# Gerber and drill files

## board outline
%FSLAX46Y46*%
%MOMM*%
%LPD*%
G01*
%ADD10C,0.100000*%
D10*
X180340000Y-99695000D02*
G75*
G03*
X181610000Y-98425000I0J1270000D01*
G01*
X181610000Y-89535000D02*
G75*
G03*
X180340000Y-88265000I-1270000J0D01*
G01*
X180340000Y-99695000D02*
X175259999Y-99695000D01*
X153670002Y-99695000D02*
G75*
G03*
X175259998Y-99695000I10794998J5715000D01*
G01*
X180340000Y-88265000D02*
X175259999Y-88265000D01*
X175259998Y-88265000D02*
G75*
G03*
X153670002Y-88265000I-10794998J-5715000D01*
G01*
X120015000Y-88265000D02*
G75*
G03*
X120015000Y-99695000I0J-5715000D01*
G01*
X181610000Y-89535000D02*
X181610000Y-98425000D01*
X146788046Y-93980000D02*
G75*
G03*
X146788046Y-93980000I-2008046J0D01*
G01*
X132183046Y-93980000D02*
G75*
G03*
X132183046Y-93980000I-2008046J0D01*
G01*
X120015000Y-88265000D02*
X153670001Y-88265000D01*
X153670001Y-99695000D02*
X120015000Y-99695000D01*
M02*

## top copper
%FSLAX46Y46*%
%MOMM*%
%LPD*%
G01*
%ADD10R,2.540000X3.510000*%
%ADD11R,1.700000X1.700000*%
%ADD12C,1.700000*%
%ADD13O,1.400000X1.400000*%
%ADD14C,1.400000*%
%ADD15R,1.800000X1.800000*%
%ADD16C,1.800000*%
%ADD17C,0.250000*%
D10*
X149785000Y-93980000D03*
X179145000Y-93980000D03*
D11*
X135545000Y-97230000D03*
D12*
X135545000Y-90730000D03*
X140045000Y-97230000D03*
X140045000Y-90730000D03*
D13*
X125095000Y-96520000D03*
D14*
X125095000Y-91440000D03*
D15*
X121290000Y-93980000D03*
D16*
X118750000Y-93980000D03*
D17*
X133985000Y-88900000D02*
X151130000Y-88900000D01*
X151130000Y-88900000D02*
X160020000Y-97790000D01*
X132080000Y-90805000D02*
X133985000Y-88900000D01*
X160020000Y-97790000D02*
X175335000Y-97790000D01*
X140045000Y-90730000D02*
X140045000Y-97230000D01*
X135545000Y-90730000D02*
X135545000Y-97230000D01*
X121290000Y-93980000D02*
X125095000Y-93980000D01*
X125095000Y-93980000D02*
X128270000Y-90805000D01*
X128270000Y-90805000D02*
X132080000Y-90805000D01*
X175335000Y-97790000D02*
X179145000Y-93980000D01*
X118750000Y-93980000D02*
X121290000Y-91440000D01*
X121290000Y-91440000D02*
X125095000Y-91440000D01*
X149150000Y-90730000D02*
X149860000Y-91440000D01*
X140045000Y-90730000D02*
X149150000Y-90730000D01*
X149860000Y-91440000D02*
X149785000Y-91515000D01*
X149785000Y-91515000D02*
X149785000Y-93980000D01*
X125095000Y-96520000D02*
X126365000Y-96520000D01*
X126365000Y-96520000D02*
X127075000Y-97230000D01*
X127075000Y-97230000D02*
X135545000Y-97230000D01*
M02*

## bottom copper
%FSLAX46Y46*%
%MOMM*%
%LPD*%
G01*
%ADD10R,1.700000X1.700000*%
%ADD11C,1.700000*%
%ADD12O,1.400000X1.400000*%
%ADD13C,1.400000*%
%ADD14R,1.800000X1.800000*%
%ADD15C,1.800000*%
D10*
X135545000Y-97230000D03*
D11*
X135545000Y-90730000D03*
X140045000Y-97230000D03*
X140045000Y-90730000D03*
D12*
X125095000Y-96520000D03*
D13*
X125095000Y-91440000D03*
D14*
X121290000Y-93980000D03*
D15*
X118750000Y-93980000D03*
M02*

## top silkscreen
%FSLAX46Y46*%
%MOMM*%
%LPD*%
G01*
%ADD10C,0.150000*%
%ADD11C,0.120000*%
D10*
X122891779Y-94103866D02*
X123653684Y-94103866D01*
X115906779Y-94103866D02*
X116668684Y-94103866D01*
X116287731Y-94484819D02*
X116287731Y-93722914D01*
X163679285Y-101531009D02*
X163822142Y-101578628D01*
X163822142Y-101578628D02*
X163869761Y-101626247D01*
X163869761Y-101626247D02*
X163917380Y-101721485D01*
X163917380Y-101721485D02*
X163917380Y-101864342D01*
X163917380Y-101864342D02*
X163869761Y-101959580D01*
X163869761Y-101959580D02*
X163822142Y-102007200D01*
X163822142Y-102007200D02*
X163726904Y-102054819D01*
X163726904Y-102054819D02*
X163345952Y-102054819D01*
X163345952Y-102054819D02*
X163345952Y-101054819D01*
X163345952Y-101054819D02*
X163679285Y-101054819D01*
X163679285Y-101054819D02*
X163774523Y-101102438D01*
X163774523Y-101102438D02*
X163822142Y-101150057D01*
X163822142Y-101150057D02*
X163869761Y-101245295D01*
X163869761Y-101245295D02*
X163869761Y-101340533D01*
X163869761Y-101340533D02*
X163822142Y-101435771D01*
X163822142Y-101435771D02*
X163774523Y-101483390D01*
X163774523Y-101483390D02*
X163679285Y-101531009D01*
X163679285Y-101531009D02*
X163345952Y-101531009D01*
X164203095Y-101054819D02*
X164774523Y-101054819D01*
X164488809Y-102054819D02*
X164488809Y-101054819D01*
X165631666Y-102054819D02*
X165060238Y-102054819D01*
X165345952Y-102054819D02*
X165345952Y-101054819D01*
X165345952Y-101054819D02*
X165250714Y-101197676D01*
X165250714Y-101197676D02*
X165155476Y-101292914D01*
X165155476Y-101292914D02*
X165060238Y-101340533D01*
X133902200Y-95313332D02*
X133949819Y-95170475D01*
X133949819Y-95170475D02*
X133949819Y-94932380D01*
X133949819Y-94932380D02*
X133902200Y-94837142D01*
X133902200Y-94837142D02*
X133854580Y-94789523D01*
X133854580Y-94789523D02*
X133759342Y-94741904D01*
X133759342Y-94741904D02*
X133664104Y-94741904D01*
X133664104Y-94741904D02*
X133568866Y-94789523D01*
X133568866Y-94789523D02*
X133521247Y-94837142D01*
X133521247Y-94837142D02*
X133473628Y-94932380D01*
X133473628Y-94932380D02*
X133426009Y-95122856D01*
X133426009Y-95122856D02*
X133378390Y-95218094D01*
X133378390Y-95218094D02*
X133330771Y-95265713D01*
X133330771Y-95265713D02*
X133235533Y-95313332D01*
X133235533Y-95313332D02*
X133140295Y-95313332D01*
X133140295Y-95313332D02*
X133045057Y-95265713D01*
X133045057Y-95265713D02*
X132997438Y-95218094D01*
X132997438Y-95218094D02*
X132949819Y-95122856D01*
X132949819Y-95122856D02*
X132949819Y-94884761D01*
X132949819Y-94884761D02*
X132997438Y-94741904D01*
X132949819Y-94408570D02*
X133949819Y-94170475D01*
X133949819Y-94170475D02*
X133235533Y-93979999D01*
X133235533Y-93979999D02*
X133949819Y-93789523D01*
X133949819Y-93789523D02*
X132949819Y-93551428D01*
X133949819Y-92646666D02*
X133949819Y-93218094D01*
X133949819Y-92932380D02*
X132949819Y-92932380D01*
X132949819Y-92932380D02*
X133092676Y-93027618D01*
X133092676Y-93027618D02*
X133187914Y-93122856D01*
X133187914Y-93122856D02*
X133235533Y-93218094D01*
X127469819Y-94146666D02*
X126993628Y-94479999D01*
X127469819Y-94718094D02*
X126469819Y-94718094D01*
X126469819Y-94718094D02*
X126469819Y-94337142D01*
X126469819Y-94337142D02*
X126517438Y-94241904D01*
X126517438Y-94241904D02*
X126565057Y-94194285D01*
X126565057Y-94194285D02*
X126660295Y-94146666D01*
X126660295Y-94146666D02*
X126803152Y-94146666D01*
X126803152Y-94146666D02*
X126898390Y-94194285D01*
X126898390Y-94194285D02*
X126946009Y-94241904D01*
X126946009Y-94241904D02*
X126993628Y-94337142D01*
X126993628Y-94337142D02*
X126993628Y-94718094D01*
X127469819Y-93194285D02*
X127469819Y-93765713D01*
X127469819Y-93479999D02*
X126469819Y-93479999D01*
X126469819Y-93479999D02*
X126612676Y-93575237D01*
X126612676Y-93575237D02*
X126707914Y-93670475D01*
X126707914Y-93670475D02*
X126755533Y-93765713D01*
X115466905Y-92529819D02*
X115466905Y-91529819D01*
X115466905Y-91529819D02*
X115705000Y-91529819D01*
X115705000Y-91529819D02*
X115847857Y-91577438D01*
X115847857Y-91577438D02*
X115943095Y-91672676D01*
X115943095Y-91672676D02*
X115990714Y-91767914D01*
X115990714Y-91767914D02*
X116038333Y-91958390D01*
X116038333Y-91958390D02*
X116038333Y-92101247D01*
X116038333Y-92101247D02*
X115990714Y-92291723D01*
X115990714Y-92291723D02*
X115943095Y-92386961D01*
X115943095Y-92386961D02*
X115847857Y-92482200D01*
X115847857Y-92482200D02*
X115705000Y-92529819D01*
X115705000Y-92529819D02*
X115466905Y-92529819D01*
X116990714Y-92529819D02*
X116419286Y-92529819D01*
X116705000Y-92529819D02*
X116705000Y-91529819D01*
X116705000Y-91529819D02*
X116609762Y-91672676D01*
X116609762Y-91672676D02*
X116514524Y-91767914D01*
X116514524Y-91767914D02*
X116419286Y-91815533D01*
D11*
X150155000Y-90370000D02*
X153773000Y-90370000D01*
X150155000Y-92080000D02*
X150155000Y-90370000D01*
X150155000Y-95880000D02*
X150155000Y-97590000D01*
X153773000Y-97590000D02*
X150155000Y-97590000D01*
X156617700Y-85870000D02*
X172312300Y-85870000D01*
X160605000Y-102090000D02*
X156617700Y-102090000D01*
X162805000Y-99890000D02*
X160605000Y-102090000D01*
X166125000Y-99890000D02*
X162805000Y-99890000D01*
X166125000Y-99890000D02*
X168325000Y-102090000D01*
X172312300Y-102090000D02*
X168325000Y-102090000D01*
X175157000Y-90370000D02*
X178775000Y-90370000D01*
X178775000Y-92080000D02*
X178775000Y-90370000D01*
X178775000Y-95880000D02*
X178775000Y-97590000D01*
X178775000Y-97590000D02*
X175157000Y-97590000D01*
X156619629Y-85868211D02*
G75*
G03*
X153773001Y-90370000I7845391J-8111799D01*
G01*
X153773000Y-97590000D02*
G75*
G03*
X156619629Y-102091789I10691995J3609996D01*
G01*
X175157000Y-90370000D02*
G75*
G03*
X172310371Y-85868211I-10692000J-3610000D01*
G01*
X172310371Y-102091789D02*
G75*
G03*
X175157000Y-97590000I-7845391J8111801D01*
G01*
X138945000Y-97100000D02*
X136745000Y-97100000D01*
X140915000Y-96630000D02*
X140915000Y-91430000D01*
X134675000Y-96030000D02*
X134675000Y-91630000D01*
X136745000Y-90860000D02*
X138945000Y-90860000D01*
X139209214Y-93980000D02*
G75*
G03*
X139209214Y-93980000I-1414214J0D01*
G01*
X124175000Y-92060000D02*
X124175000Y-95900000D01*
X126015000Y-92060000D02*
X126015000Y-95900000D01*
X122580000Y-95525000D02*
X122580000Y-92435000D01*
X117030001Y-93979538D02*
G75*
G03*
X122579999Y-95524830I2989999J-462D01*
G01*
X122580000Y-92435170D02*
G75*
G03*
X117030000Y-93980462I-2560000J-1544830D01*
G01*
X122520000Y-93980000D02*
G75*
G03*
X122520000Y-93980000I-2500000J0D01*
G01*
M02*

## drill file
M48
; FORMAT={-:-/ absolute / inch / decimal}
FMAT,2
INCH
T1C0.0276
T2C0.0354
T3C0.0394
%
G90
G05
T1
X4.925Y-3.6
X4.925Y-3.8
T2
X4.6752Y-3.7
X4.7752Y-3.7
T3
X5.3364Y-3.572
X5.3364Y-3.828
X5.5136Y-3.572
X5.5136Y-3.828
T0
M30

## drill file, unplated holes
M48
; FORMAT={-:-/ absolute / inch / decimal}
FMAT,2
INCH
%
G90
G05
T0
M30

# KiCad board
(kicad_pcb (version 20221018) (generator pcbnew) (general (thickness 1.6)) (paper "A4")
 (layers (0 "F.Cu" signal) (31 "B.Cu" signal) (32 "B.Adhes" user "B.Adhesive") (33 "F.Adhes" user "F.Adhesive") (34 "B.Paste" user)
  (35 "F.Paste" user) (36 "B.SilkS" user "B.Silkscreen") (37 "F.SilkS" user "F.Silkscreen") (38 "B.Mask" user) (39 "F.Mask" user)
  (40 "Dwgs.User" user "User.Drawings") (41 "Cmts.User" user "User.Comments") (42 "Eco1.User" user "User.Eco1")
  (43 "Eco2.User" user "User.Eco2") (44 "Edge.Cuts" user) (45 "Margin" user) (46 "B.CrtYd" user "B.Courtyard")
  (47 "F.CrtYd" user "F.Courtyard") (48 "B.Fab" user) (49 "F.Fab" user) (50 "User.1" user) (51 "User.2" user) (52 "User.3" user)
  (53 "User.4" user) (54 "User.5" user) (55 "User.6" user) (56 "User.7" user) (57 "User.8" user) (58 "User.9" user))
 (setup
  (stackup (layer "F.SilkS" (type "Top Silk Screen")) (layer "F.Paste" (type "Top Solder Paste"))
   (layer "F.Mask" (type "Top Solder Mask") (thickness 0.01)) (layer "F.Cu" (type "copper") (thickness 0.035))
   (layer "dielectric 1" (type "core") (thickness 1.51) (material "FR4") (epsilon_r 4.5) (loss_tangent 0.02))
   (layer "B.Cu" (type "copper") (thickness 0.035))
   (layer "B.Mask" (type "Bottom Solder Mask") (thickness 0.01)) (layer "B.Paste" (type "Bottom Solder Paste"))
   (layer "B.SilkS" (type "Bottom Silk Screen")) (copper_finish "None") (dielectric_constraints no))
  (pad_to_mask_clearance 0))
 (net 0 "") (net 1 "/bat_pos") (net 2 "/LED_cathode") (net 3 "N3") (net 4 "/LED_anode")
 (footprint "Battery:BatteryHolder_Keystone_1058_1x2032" (layer "F.Cu") (at 164.465 93.98)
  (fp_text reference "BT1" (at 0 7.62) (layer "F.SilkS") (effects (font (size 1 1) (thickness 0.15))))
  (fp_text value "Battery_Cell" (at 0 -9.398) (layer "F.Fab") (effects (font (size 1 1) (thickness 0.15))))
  (fp_line (start -14.31 -3.61) (end -10.692 -3.61) (stroke (width 0.12) (type solid)) (layer "F.SilkS"))
  (fp_line (start -14.31 -1.9) (end -14.31 -3.61) (stroke (width 0.12) (type solid)) (layer "F.SilkS"))
  (fp_line (start -14.31 1.9) (end -14.31 3.61) (stroke (width 0.12) (type solid)) (layer "F.SilkS"))
  (fp_line (start -10.692 3.61) (end -14.31 3.61) (stroke (width 0.12) (type solid)) (layer "F.SilkS"))
  (fp_line (start -7.8473 -8.11) (end 7.8473 -8.11) (stroke (width 0.12) (type solid)) (layer "F.SilkS"))
  (fp_line (start -3.86 8.11) (end -7.8473 8.11) (stroke (width 0.12) (type solid)) (layer "F.SilkS"))
  (fp_line (start -1.66 5.91) (end -3.86 8.11) (stroke (width 0.12) (type solid)) (layer "F.SilkS"))
  (fp_line (start 1.66 5.91) (end -1.66 5.91) (stroke (width 0.12) (type solid)) (layer "F.SilkS"))
  (fp_line (start 1.66 5.91) (end 3.86 8.11) (stroke (width 0.12) (type solid)) (layer "F.SilkS"))
  (fp_line (start 7.8473 8.11) (end 3.86 8.11) (stroke (width 0.12) (type solid)) (layer "F.SilkS"))
  (fp_line (start 10.692 -3.61) (end 14.31 -3.61) (stroke (width 0.12) (type solid)) (layer "F.SilkS"))
  (fp_line (start 14.31 -1.9) (end 14.31 -3.61) (stroke (width 0.12) (type solid)) (layer "F.SilkS"))
  (fp_line (start 14.31 1.9) (end 14.31 3.61) (stroke (width 0.12) (type solid)) (layer "F.SilkS"))
  (fp_line (start 14.31 3.61) (end 10.692 3.61) (stroke (width 0.12) (type solid)) (layer "F.SilkS"))
  (fp_arc (start -10.692 -3.61) (mid -9.538084 -6.031244) (end -7.845371 -8.111789) (stroke (width 0.12) (type solid)) (layer "F.SilkS"))
  (fp_arc (start -7.845371 8.111789) (mid -9.538085 6.031244) (end -10.692 3.61) (stroke (width 0.12) (type solid)) (layer "F.SilkS"))
  (fp_arc (start 7.845371 -8.111789) (mid 9.538085 -6.031244) (end 10.692 -3.61) (stroke (width 0.12) (type solid)) (layer "F.SilkS"))
  (fp_arc (start 10.692 3.61) (mid 9.538084 6.031244) (end 7.845371 8.111789) (stroke (width 0.12) (type solid)) (layer "F.SilkS"))
  (pad "1" smd rect (at -14.68 0) (size 2.54 3.51) (layers "F.Cu" "F.Paste" "F.Mask") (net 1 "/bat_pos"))
  (pad "2" smd rect (at 14.68 0) (size 2.54 3.51) (layers "F.Cu" "F.Paste" "F.Mask") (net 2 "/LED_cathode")))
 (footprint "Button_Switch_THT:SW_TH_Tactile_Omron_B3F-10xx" (layer "F.Cu") (at 135.545 97.23 90)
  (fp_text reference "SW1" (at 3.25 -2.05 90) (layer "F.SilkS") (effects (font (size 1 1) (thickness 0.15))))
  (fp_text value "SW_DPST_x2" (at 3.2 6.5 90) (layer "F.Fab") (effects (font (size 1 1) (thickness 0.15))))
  (fp_line (start 0.13 3.4) (end 0.13 1.2) (stroke (width 0.12) (type solid)) (layer "F.SilkS"))
  (fp_line (start 0.6 5.37) (end 5.8 5.37) (stroke (width 0.12) (type solid)) (layer "F.SilkS"))
  (fp_line (start 1.2 -0.87) (end 5.6 -0.87) (stroke (width 0.12) (type solid)) (layer "F.SilkS"))
  (fp_line (start 6.37 1.2) (end 6.37 3.4) (stroke (width 0.12) (type solid)) (layer "F.SilkS"))
  (fp_circle (center 3.25 2.25) (end 4.25 3.25) (stroke (width 0.12) (type solid)) (fill none) (layer "F.SilkS"))
  (pad "1" thru_hole rect (at 0 0 90) (size 1.7 1.7) (drill 1) (layers "*.Cu" "*.Mask") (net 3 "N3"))
  (pad "1" thru_hole circle (at 6.5 0 90) (size 1.7 1.7) (drill 1) (layers "*.Cu" "*.Mask") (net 3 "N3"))
  (pad "2" thru_hole circle (at 0 4.5 90) (size 1.7 1.7) (drill 1) (layers "*.Cu" "*.Mask") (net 1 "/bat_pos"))
  (pad "2" thru_hole circle (at 6.5 4.5 90) (size 1.7 1.7) (drill 1) (layers "*.Cu" "*.Mask") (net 1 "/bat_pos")))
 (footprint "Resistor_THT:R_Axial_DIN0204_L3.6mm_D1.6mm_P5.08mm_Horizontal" (layer "F.Cu") (at 125.095 91.44 -90)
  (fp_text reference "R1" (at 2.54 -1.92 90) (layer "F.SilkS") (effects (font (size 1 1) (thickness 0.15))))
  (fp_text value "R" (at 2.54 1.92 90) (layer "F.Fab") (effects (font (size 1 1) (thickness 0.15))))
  (fp_line (start 0.62 -0.92) (end 4.46 -0.92) (stroke (width 0.12) (type solid)) (layer "F.SilkS"))
  (fp_line (start 0.62 0.92) (end 4.46 0.92) (stroke (width 0.12) (type solid)) (layer "F.SilkS"))
  (pad "1" thru_hole circle (at 0 0 270) (size 1.4 1.4) (drill 0.7) (layers "*.Cu" "*.Mask") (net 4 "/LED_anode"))
  (pad "2" thru_hole oval (at 5.08 0 270) (size 1.4 1.4) (drill 0.7) (layers "*.Cu" "*.Mask") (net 3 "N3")))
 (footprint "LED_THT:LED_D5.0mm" (layer "F.Cu") (at 121.29 93.98 180)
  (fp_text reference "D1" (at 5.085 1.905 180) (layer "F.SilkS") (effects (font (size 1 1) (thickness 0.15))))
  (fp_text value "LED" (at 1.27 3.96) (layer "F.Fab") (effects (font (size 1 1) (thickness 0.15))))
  (fp_line (start -1.29 -1.545) (end -1.29 1.545) (stroke (width 0.12) (type solid)) (layer "F.SilkS"))
  (fp_arc (start -1.29 -1.54483) (mid 2.072002 -2.880433) (end 4.26 0.000462) (stroke (width 0.12) (type solid)) (layer "F.SilkS"))
  (fp_arc (start 4.26 -0.000462) (mid 2.072002 2.880433) (end -1.29 1.54483) (stroke (width 0.12) (type solid)) (layer "F.SilkS"))
  (fp_circle (center 1.27 0) (end 3.77 0) (stroke (width 0.12) (type solid)) (fill none) (layer "F.SilkS"))
  (pad "1" thru_hole rect (at 0 0 180) (size 1.8 1.8) (drill 0.9) (layers "*.Cu" "*.Mask") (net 2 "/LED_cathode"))
  (pad "2" thru_hole circle (at 2.54 0 180) (size 1.8 1.8) (drill 0.9) (layers "*.Cu" "*.Mask") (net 4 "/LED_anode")))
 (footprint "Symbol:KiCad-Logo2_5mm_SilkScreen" (layer "B.Cu") (at 164.465 93.98 180)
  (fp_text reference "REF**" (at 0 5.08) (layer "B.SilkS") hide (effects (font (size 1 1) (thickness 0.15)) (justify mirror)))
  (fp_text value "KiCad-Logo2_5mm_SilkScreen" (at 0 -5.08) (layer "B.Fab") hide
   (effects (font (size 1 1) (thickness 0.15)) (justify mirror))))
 (gr_line (start 153.670001 99.695) (end 120.015 99.695) (stroke (width 0.1) (type default)) (layer "Edge.Cuts"))
 (gr_arc (start 180.34 88.265) (mid 181.238026 88.636974) (end 181.61 89.535) (stroke (width 0.1) (type default)) (layer "Edge.Cuts"))
 (gr_line (start 120.015 88.265) (end 153.670001 88.265) (stroke (width 0.1) (type default)) (layer "Edge.Cuts"))
 (gr_arc (start 175.259999 99.695) (mid 164.465 106.194468) (end 153.670001 99.695) (stroke (width 0.1) (type default)) (layer "Edge.Cuts"))
 (gr_arc (start 181.61 98.425) (mid 181.238026 99.323026) (end 180.34 99.695) (stroke (width 0.1) (type default)) (layer "Edge.Cuts"))
 (gr_circle (center 144.78 93.98) (end 146.685 94.615) (stroke (width 0.1) (type default)) (fill none) (layer "Edge.Cuts"))
 (gr_line (start 181.61 89.535) (end 181.61 98.425) (stroke (width 0.1) (type default)) (layer "Edge.Cuts"))
 (gr_arc (start 153.670001 88.265) (mid 164.465 81.765532) (end 175.259999 88.265) (stroke (width 0.1) (type default)) (layer "Edge.Cuts"))
 (gr_line (start 180.34 88.265) (end 175.259999 88.265) (stroke (width 0.1) (type default)) (layer "Edge.Cuts"))
 (gr_circle (center 130.175 93.98) (end 132.08 94.615) (stroke (width 0.1) (type default)) (fill none) (layer "Edge.Cuts"))
 (gr_arc (start 120.015 99.695) (mid 114.3 93.98) (end 120.015 88.265) (stroke (width 0.1) (type default)) (layer "Edge.Cuts"))
 (gr_line (start 180.34 99.695) (end 175.259999 99.695) (stroke (width 0.1) (type default)) (layer "Edge.Cuts"))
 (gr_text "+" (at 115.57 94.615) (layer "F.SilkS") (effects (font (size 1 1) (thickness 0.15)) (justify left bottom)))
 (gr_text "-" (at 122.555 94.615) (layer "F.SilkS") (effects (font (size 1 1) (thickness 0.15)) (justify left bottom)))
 (segment (start 140.045 90.73) (end 140.045 97.23) (width 0.25) (layer "F.Cu") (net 1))
 (segment (start 140.045 90.73) (end 149.15 90.73) (width 0.25) (layer "F.Cu") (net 1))
 (segment (start 149.15 90.73) (end 149.86 91.44) (width 0.25) (layer "F.Cu") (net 1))
 (segment (start 149.785 91.515) (end 149.785 93.98) (width 0.25) (layer "F.Cu") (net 1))
 (segment (start 149.86 91.44) (end 149.785 91.515) (width 0.25) (layer "F.Cu") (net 1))
 (segment (start 128.27 90.805) (end 132.08 90.805) (width 0.25) (layer "F.Cu") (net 2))
 (segment (start 160.02 97.79) (end 175.335 97.79) (width 0.25) (layer "F.Cu") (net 2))
 (segment (start 133.985 88.9) (end 151.13 88.9) (width 0.25) (layer "F.Cu") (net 2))
 (segment (start 151.13 88.9) (end 160.02 97.79) (width 0.25) (layer "F.Cu") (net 2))
 (segment (start 125.095 93.98) (end 128.27 90.805) (width 0.25) (layer "F.Cu") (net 2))
 (segment (start 132.08 90.805) (end 133.985 88.9) (width 0.25) (layer "F.Cu") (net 2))
 (segment (start 121.29 93.98) (end 125.095 93.98) (width 0.25) (layer "F.Cu") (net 2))
 (segment (start 175.335 97.79) (end 179.145 93.98) (width 0.25) (layer "F.Cu") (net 2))
 (segment (start 121.29 91.44) (end 125.095 91.44) (width 0.25) (layer "F.Cu") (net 4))
 (segment (start 118.75 93.98) (end 121.29 91.44) (width 0.25) (layer "F.Cu") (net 4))
 (segment (start 127.075 97.23) (end 135.545 97.23) (width 0.25) (layer "F.Cu") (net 3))
 (segment (start 125.095 96.52) (end 126.365 96.52) (width 0.25) (layer "F.Cu") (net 3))
 (segment (start 126.365 96.52) (end 127.075 97.23) (width 0.25) (layer "F.Cu") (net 3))
 (segment (start 135.545 90.73) (end 135.545 97.23) (width 0.25) (layer "F.Cu") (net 3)))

